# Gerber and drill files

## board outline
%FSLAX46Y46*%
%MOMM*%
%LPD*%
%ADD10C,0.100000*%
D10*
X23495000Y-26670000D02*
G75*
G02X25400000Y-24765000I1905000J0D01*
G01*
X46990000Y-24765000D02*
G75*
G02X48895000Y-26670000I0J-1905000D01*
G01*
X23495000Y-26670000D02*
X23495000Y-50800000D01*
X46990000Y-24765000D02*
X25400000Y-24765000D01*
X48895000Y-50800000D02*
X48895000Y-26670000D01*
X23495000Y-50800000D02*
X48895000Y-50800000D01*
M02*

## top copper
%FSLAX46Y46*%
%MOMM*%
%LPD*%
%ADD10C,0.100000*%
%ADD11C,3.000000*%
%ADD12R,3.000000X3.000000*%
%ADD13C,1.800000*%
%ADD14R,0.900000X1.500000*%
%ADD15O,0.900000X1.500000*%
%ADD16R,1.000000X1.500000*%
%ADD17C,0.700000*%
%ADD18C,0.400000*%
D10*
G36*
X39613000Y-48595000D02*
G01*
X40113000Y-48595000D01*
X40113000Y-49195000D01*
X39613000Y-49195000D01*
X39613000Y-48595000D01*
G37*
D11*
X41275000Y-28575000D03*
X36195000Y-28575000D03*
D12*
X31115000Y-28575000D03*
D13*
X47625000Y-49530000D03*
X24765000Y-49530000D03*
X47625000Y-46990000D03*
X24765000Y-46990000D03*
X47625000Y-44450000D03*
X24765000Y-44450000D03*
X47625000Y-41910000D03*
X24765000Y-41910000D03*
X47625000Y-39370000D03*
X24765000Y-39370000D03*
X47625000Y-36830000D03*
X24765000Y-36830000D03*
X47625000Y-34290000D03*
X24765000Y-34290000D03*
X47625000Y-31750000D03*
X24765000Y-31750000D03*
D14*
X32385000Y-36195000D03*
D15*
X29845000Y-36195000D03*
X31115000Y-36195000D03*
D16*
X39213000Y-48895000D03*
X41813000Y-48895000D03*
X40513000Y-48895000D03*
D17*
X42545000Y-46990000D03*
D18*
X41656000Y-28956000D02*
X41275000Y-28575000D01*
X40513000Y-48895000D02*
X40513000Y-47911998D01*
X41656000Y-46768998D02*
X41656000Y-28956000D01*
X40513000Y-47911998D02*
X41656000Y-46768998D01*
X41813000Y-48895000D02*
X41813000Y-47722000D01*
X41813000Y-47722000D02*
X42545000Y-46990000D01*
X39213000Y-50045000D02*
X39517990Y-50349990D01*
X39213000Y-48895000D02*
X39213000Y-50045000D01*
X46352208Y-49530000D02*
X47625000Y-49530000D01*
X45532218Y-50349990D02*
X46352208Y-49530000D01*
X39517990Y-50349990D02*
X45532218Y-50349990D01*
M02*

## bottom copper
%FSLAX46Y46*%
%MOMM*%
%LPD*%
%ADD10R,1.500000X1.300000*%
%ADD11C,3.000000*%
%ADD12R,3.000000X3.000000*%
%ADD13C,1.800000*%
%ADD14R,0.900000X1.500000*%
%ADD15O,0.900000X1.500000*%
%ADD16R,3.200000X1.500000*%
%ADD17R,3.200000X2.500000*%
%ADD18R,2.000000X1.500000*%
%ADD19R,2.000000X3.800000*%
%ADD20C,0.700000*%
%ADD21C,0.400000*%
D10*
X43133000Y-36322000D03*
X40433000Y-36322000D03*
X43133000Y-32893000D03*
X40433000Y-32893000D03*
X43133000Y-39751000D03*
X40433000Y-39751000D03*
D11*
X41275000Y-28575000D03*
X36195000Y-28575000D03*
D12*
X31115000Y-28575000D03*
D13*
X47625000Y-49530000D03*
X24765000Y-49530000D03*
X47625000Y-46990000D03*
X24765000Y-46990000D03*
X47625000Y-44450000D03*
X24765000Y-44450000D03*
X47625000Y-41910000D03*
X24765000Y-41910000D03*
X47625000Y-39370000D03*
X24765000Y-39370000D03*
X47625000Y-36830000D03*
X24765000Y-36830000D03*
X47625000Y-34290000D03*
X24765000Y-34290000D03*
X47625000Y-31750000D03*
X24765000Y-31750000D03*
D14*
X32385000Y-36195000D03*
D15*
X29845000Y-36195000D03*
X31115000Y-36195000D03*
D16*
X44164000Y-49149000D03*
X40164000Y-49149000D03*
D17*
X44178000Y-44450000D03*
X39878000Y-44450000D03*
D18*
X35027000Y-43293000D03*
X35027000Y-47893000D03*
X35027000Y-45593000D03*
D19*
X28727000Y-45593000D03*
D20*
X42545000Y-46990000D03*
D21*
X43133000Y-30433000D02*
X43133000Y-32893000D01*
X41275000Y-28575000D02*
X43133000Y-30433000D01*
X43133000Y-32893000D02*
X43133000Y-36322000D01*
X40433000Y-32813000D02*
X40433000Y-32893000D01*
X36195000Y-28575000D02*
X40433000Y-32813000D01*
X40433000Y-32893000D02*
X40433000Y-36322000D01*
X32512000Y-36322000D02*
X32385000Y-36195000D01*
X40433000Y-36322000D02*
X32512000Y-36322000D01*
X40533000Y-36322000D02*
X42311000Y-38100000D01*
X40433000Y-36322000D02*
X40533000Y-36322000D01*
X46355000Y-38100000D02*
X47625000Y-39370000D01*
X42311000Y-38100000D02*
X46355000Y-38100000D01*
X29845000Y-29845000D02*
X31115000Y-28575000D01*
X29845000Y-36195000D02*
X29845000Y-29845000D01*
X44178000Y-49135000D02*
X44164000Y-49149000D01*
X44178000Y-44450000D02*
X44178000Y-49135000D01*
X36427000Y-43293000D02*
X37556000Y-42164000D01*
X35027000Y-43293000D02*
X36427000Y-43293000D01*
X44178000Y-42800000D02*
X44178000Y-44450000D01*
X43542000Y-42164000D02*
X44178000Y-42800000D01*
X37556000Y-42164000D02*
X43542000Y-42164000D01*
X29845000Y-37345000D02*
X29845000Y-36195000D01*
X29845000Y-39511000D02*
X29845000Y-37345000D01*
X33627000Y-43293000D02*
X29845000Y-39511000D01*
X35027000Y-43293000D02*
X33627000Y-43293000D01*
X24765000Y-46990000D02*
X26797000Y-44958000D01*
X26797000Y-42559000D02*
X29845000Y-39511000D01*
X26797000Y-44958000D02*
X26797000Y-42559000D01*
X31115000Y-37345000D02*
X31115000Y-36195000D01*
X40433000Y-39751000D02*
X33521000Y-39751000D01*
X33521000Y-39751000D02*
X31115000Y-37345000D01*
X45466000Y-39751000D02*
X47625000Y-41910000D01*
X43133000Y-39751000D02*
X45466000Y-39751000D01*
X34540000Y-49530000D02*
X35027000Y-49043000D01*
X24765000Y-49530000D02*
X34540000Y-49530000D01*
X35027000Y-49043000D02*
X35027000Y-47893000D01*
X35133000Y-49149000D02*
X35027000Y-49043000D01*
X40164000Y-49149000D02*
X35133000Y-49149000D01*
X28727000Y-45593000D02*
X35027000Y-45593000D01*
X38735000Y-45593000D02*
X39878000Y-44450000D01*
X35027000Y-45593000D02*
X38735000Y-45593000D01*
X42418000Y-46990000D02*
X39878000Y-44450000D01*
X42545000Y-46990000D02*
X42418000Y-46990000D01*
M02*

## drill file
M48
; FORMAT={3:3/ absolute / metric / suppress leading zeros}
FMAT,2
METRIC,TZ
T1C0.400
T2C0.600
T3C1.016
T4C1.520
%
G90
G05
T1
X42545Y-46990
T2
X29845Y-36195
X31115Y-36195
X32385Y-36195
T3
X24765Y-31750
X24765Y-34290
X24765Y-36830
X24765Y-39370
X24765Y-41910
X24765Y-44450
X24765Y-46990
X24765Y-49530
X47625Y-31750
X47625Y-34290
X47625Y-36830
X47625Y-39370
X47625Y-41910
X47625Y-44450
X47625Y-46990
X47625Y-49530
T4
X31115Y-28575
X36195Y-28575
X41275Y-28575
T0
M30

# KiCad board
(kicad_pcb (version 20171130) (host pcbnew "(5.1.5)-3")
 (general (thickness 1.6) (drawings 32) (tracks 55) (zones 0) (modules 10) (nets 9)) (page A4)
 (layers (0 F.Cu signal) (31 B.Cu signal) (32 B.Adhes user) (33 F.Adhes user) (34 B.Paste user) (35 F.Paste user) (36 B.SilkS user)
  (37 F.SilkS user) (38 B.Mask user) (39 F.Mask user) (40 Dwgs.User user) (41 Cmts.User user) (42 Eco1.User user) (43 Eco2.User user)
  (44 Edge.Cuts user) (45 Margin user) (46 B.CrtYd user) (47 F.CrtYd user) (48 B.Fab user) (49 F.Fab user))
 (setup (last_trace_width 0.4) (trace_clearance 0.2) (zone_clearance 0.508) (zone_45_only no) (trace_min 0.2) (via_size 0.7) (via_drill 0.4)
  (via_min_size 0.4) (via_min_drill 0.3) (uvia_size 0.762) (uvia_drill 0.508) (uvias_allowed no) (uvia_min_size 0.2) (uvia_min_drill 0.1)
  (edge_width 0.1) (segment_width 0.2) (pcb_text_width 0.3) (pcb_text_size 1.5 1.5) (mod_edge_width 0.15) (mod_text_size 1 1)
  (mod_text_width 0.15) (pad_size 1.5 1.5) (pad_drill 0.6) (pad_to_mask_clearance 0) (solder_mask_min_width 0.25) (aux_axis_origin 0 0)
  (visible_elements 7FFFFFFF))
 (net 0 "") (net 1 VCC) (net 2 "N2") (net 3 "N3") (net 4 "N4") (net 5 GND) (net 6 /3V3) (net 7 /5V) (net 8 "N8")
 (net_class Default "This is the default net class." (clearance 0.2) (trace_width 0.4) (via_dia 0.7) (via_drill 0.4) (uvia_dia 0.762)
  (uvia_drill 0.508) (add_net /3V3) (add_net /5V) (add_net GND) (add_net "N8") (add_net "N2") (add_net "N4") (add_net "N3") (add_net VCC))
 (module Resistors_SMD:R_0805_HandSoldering (layer B.Cu) (at 41.783 36.322 180)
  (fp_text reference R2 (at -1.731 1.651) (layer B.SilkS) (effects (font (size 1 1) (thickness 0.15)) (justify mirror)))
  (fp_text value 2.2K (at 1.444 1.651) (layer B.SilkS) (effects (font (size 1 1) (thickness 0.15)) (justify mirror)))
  (pad 1 smd rect (at -1.35 0 180) (size 1.5 1.3) (layers B.Cu B.Paste B.Mask) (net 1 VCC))
  (pad 2 smd rect (at 1.35 0 180) (size 1.5 1.3) (layers B.Cu B.Paste B.Mask) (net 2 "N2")))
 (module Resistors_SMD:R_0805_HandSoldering (layer B.Cu) (at 41.783 32.893 180)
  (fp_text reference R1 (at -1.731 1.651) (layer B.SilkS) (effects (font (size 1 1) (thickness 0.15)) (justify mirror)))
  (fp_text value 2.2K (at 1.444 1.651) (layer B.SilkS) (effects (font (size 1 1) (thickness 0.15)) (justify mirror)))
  (pad 1 smd rect (at -1.35 0 180) (size 1.5 1.3) (layers B.Cu B.Paste B.Mask) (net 1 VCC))
  (pad 2 smd rect (at 1.35 0 180) (size 1.5 1.3) (layers B.Cu B.Paste B.Mask) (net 2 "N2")))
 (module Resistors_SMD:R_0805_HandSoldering (layer B.Cu) (at 41.783 39.751 180)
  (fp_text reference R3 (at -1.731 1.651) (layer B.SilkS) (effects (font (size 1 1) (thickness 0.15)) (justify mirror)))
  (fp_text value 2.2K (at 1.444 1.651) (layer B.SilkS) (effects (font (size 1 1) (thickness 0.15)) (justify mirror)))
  (pad 1 smd rect (at -1.35 0 180) (size 1.5 1.3) (layers B.Cu B.Paste B.Mask) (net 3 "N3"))
  (pad 2 smd rect (at 1.35 0 180) (size 1.5 1.3) (layers B.Cu B.Paste B.Mask) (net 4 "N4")))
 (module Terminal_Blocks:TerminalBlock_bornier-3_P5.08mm (layer F.Cu) (at 31.115 28.575)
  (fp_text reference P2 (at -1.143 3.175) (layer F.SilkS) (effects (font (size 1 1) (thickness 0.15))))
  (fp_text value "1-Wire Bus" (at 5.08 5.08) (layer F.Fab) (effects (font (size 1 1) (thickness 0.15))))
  (pad 3 thru_hole circle (at 10.16 0) (size 3 3) (drill 1.52) (layers *.Cu *.Mask) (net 1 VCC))
  (pad 2 thru_hole circle (at 5.08 0) (size 3 3) (drill 1.52) (layers *.Cu *.Mask) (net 2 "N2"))
  (pad 1 thru_hole rect (at 0 0) (size 3 3) (drill 1.52) (layers *.Cu *.Mask) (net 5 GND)))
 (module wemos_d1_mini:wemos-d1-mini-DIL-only (layer B.Cu) (at 36.195 40.64 90)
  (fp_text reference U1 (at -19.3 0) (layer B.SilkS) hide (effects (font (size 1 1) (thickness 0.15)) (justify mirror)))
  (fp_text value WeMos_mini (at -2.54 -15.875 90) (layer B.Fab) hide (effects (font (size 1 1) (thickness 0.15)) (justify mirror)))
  (pad 16 thru_hole circle (at -8.89 11.43 90) (size 1.8 1.8) (drill 1.016) (layers *.Cu *.Mask) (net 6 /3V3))
  (pad 1 thru_hole circle (at -8.89 -11.43 90) (size 1.8 1.8) (drill 1.016) (layers *.Cu *.Mask) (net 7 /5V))
  (pad 15 thru_hole circle (at -6.35 11.43 90) (size 1.8 1.8) (drill 1.016) (layers *.Cu *.Mask))
  (pad 2 thru_hole circle (at -6.35 -11.43 90) (size 1.8 1.8) (drill 1.016) (layers *.Cu *.Mask) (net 5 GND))
  (pad 14 thru_hole circle (at -3.81 11.43 90) (size 1.8 1.8) (drill 1.016) (layers *.Cu *.Mask))
  (pad 3 thru_hole circle (at -3.81 -11.43 90) (size 1.8 1.8) (drill 1.016) (layers *.Cu *.Mask))
  (pad 13 thru_hole circle (at -1.27 11.43 90) (size 1.8 1.8) (drill 1.016) (layers *.Cu *.Mask) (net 3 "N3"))
  (pad 4 thru_hole circle (at -1.27 -11.43 90) (size 1.8 1.8) (drill 1.016) (layers *.Cu *.Mask))
  (pad 12 thru_hole circle (at 1.27 11.43 90) (size 1.8 1.8) (drill 1.016) (layers *.Cu *.Mask) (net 2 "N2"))
  (pad 5 thru_hole circle (at 1.27 -11.43 90) (size 1.8 1.8) (drill 1.016) (layers *.Cu *.Mask))
  (pad 11 thru_hole circle (at 3.81 11.43 90) (size 1.8 1.8) (drill 1.016) (layers *.Cu *.Mask))
  (pad 6 thru_hole circle (at 3.81 -11.43 90) (size 1.8 1.8) (drill 1.016) (layers *.Cu *.Mask))
  (pad 10 thru_hole circle (at 6.35 11.43 90) (size 1.8 1.8) (drill 1.016) (layers *.Cu *.Mask))
  (pad 7 thru_hole circle (at 6.35 -11.43 90) (size 1.8 1.8) (drill 1.016) (layers *.Cu *.Mask))
  (pad 9 thru_hole circle (at 8.89 11.43 90) (size 1.8 1.8) (drill 1.016) (layers *.Cu *.Mask))
  (pad 8 thru_hole circle (at 8.89 -11.43 90) (size 1.8 1.8) (drill 1.016) (layers *.Cu *.Mask)))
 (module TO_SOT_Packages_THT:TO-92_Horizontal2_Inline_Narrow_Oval (layer F.Cu) (at 32.385 36.195 180)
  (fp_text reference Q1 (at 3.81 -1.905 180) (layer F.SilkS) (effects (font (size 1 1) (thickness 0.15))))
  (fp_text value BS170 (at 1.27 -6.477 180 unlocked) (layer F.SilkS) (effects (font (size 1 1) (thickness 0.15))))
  (pad 1 thru_hole rect (at 0 0) (size 0.9 1.5) (drill 0.6) (layers *.Cu *.Mask) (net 2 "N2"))
  (pad 3 thru_hole oval (at 2.54 0) (size 0.9 1.5) (drill 0.6) (layers *.Cu *.Mask) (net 5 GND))
  (pad 2 thru_hole oval (at 1.27 0) (size 0.9 1.5) (drill 0.6) (layers *.Cu *.Mask) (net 4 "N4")))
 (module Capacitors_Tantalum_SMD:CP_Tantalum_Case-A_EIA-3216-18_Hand (layer B.Cu) (at 42.164 49.149)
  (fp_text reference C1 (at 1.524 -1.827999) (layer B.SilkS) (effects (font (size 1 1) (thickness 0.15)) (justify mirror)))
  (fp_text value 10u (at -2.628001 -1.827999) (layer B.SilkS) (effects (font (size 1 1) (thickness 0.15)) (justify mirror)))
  (pad 2 smd rect (at 2 0) (size 3.2 1.5) (layers B.Cu B.Paste B.Mask) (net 5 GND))
  (pad 1 smd rect (at -2 0) (size 3.2 1.5) (layers B.Cu B.Paste B.Mask) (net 7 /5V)))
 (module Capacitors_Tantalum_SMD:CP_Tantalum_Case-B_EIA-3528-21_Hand (layer B.Cu) (at 42.028 44.45)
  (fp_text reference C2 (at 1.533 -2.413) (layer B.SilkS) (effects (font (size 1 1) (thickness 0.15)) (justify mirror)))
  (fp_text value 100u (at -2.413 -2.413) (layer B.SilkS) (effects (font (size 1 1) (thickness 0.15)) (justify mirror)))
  (pad 2 smd rect (at 2.15 0) (size 3.2 2.5) (layers B.Cu B.Paste B.Mask) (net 5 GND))
  (pad 1 smd rect (at -2.15 0) (size 3.2 2.5) (layers B.Cu B.Paste B.Mask) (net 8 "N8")))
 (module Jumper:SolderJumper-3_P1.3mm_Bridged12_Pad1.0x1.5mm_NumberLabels (layer F.Cu) (at 40.513 48.895)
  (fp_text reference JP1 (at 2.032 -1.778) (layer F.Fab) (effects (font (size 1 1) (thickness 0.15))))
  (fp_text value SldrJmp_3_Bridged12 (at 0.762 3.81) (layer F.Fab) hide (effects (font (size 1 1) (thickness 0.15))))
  (fp_poly (pts (xy -0.9 -0.3) (xy -0.4 -0.3) (xy -0.4 0.3) (xy -0.9 0.3)) (layer F.Cu) (width 0))
  (pad 1 smd rect (at -1.3 0) (size 1 1.5) (layers F.Cu F.Mask) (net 6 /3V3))
  (pad 3 smd rect (at 1.3 0) (size 1 1.5) (layers F.Cu F.Mask) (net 8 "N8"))
  (pad 2 smd rect (at 0 0) (size 1 1.5) (layers F.Cu F.Mask) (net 1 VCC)))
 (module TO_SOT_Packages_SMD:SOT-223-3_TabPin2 (layer B.Cu) (at 31.877 45.593 180)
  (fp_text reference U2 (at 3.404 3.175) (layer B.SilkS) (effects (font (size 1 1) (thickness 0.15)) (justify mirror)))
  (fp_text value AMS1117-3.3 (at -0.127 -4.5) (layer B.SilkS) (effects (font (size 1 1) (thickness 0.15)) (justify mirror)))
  (pad 1 smd rect (at -3.15 2.3 180) (size 2 1.5) (layers B.Cu B.Paste B.Mask) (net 5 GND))
  (pad 3 smd rect (at -3.15 -2.3 180) (size 2 1.5) (layers B.Cu B.Paste B.Mask) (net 7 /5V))
  (pad 2 smd rect (at -3.15 0 180) (size 2 1.5) (layers B.Cu B.Paste B.Mask) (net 8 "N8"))
  (pad 2 smd rect (at 3.15 0 180) (size 2 3.8) (layers B.Cu B.Paste B.Mask) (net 8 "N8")))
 (gr_arc (start 25.4 26.67) (end 25.4 24.765) (angle -90) (layer Edge.Cuts) (width 0.1))
 (gr_arc (start 46.99 26.67) (end 48.895 26.67) (angle -90) (layer Edge.Cuts) (width 0.1))
 (gr_line (start 23.495 26.67) (end 23.495 50.8) (layer Edge.Cuts) (width 0.1))
 (gr_line (start 46.99 24.765) (end 25.4 24.765) (layer Edge.Cuts) (width 0.1))
 (gr_line (start 48.895 50.8) (end 48.895 26.67) (layer Edge.Cuts) (width 0.1))
 (gr_line (start 23.495 50.8) (end 48.895 50.8) (layer Edge.Cuts) (width 0.1))
 (segment (start 43.133 30.433) (end 43.133 32.893) (width 0.4) (layer B.Cu) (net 1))
 (segment (start 41.275 28.575) (end 43.133 30.433) (width 0.4) (layer B.Cu) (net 1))
 (segment (start 43.133 32.893) (end 43.133 36.322) (width 0.4) (layer B.Cu) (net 1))
 (segment (start 41.656 28.956) (end 41.275 28.575) (width 0.4) (layer F.Cu) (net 1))
 (segment (start 40.513 48.895) (end 40.513 47.911998) (width 0.4) (layer F.Cu) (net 1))
 (segment (start 41.656 46.768998) (end 41.656 28.956) (width 0.4) (layer F.Cu) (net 1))
 (segment (start 40.513 47.911998) (end 41.656 46.768998) (width 0.4) (layer F.Cu) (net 1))
 (segment (start 40.433 32.813) (end 40.433 32.893) (width 0.4) (layer B.Cu) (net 2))
 (segment (start 36.195 28.575) (end 40.433 32.813) (width 0.4) (layer B.Cu) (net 2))
 (segment (start 40.433 32.893) (end 40.433 36.322) (width 0.4) (layer B.Cu) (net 2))
 (segment (start 32.512 36.322) (end 32.385 36.195) (width 0.4) (layer B.Cu) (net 2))
 (segment (start 40.433 36.322) (end 32.512 36.322) (width 0.4) (layer B.Cu) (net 2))
 (segment (start 40.533 36.322) (end 42.311 38.1) (width 0.4) (layer B.Cu) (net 2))
 (segment (start 40.433 36.322) (end 40.533 36.322) (width 0.4) (layer B.Cu) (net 2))
 (segment (start 46.355 38.1) (end 47.625 39.37) (width 0.4) (layer B.Cu) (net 2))
 (segment (start 42.311 38.1) (end 46.355 38.1) (width 0.4) (layer B.Cu) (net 2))
 (segment (start 29.845 29.845) (end 31.115 28.575) (width 0.4) (layer B.Cu) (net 5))
 (segment (start 29.845 36.195) (end 29.845 29.845) (width 0.4) (layer B.Cu) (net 5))
 (segment (start 44.178 49.135) (end 44.164 49.149) (width 0.4) (layer B.Cu) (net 5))
 (segment (start 44.178 44.45) (end 44.178 49.135) (width 0.4) (layer B.Cu) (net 5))
 (segment (start 36.427 43.293) (end 37.556 42.164) (width 0.4) (layer B.Cu) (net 5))
 (segment (start 35.027 43.293) (end 36.427 43.293) (width 0.4) (layer B.Cu) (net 5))
 (segment (start 44.178 42.8) (end 44.178 44.45) (width 0.4) (layer B.Cu) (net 5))
 (segment (start 43.542 42.164) (end 44.178 42.8) (width 0.4) (layer B.Cu) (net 5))
 (segment (start 37.556 42.164) (end 43.542 42.164) (width 0.4) (layer B.Cu) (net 5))
 (segment (start 29.845 37.345) (end 29.845 36.195) (width 0.4) (layer B.Cu) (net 5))
 (segment (start 29.845 39.511) (end 29.845 37.345) (width 0.4) (layer B.Cu) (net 5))
 (segment (start 33.627 43.293) (end 29.845 39.511) (width 0.4) (layer B.Cu) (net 5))
 (segment (start 35.027 43.293) (end 33.627 43.293) (width 0.4) (layer B.Cu) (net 5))
 (segment (start 24.765 46.99) (end 26.797 44.958) (width 0.4) (layer B.Cu) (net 5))
 (segment (start 26.797 42.559) (end 29.845 39.511) (width 0.4) (layer B.Cu) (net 5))
 (segment (start 26.797 44.958) (end 26.797 42.559) (width 0.4) (layer B.Cu) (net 5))
 (segment (start 31.115 37.345) (end 31.115 36.195) (width 0.4) (layer B.Cu) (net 4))
 (segment (start 40.433 39.751) (end 33.521 39.751) (width 0.4) (layer B.Cu) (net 4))
 (segment (start 33.521 39.751) (end 31.115 37.345) (width 0.4) (layer B.Cu) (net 4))
 (segment (start 45.466 39.751) (end 47.625 41.91) (width 0.4) (layer B.Cu) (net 3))
 (segment (start 43.133 39.751) (end 45.466 39.751) (width 0.4) (layer B.Cu) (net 3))
 (segment (start 34.54 49.53) (end 35.027 49.043) (width 0.4) (layer B.Cu) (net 7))
 (segment (start 24.765 49.53) (end 34.54 49.53) (width 0.4) (layer B.Cu) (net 7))
 (segment (start 35.027 49.043) (end 35.027 47.893) (width 0.4) (layer B.Cu) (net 7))
 (segment (start 35.133 49.149) (end 35.027 49.043) (width 0.4) (layer B.Cu) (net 7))
 (segment (start 40.164 49.149) (end 35.133 49.149) (width 0.4) (layer B.Cu) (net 7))
 (segment (start 28.727 45.593) (end 35.027 45.593) (width 0.4) (layer B.Cu) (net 8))
 (segment (start 38.735 45.593) (end 39.878 44.45) (width 0.4) (layer B.Cu) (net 8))
 (segment (start 35.027 45.593) (end 38.735 45.593) (width 0.4) (layer B.Cu) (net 8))
 (segment (start 41.813 48.895) (end 41.813 47.722) (width 0.4) (layer F.Cu) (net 8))
 (via (at 42.545 46.99) (size 0.7) (drill 0.4) (layers F.Cu B.Cu) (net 8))
 (segment (start 41.813 47.722) (end 42.545 46.99) (width 0.4) (layer F.Cu) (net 8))
 (segment (start 42.418 46.99) (end 39.878 44.45) (width 0.4) (layer B.Cu) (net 8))
 (segment (start 42.545 46.99) (end 42.418 46.99) (width 0.4) (layer B.Cu) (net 8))
 (segment (start 39.213 50.045) (end 39.51799 50.34999) (width 0.4) (layer F.Cu) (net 6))
 (segment (start 39.213 48.895) (end 39.213 50.045) (width 0.4) (layer F.Cu) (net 6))
 (segment (start 46.352208 49.53) (end 47.625 49.53) (width 0.4) (layer F.Cu) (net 6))
 (segment (start 45.532218 50.34999) (end 46.352208 49.53) (width 0.4) (layer F.Cu) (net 6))
 (segment (start 39.51799 50.34999) (end 45.532218 50.34999) (width 0.4) (layer F.Cu) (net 6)))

